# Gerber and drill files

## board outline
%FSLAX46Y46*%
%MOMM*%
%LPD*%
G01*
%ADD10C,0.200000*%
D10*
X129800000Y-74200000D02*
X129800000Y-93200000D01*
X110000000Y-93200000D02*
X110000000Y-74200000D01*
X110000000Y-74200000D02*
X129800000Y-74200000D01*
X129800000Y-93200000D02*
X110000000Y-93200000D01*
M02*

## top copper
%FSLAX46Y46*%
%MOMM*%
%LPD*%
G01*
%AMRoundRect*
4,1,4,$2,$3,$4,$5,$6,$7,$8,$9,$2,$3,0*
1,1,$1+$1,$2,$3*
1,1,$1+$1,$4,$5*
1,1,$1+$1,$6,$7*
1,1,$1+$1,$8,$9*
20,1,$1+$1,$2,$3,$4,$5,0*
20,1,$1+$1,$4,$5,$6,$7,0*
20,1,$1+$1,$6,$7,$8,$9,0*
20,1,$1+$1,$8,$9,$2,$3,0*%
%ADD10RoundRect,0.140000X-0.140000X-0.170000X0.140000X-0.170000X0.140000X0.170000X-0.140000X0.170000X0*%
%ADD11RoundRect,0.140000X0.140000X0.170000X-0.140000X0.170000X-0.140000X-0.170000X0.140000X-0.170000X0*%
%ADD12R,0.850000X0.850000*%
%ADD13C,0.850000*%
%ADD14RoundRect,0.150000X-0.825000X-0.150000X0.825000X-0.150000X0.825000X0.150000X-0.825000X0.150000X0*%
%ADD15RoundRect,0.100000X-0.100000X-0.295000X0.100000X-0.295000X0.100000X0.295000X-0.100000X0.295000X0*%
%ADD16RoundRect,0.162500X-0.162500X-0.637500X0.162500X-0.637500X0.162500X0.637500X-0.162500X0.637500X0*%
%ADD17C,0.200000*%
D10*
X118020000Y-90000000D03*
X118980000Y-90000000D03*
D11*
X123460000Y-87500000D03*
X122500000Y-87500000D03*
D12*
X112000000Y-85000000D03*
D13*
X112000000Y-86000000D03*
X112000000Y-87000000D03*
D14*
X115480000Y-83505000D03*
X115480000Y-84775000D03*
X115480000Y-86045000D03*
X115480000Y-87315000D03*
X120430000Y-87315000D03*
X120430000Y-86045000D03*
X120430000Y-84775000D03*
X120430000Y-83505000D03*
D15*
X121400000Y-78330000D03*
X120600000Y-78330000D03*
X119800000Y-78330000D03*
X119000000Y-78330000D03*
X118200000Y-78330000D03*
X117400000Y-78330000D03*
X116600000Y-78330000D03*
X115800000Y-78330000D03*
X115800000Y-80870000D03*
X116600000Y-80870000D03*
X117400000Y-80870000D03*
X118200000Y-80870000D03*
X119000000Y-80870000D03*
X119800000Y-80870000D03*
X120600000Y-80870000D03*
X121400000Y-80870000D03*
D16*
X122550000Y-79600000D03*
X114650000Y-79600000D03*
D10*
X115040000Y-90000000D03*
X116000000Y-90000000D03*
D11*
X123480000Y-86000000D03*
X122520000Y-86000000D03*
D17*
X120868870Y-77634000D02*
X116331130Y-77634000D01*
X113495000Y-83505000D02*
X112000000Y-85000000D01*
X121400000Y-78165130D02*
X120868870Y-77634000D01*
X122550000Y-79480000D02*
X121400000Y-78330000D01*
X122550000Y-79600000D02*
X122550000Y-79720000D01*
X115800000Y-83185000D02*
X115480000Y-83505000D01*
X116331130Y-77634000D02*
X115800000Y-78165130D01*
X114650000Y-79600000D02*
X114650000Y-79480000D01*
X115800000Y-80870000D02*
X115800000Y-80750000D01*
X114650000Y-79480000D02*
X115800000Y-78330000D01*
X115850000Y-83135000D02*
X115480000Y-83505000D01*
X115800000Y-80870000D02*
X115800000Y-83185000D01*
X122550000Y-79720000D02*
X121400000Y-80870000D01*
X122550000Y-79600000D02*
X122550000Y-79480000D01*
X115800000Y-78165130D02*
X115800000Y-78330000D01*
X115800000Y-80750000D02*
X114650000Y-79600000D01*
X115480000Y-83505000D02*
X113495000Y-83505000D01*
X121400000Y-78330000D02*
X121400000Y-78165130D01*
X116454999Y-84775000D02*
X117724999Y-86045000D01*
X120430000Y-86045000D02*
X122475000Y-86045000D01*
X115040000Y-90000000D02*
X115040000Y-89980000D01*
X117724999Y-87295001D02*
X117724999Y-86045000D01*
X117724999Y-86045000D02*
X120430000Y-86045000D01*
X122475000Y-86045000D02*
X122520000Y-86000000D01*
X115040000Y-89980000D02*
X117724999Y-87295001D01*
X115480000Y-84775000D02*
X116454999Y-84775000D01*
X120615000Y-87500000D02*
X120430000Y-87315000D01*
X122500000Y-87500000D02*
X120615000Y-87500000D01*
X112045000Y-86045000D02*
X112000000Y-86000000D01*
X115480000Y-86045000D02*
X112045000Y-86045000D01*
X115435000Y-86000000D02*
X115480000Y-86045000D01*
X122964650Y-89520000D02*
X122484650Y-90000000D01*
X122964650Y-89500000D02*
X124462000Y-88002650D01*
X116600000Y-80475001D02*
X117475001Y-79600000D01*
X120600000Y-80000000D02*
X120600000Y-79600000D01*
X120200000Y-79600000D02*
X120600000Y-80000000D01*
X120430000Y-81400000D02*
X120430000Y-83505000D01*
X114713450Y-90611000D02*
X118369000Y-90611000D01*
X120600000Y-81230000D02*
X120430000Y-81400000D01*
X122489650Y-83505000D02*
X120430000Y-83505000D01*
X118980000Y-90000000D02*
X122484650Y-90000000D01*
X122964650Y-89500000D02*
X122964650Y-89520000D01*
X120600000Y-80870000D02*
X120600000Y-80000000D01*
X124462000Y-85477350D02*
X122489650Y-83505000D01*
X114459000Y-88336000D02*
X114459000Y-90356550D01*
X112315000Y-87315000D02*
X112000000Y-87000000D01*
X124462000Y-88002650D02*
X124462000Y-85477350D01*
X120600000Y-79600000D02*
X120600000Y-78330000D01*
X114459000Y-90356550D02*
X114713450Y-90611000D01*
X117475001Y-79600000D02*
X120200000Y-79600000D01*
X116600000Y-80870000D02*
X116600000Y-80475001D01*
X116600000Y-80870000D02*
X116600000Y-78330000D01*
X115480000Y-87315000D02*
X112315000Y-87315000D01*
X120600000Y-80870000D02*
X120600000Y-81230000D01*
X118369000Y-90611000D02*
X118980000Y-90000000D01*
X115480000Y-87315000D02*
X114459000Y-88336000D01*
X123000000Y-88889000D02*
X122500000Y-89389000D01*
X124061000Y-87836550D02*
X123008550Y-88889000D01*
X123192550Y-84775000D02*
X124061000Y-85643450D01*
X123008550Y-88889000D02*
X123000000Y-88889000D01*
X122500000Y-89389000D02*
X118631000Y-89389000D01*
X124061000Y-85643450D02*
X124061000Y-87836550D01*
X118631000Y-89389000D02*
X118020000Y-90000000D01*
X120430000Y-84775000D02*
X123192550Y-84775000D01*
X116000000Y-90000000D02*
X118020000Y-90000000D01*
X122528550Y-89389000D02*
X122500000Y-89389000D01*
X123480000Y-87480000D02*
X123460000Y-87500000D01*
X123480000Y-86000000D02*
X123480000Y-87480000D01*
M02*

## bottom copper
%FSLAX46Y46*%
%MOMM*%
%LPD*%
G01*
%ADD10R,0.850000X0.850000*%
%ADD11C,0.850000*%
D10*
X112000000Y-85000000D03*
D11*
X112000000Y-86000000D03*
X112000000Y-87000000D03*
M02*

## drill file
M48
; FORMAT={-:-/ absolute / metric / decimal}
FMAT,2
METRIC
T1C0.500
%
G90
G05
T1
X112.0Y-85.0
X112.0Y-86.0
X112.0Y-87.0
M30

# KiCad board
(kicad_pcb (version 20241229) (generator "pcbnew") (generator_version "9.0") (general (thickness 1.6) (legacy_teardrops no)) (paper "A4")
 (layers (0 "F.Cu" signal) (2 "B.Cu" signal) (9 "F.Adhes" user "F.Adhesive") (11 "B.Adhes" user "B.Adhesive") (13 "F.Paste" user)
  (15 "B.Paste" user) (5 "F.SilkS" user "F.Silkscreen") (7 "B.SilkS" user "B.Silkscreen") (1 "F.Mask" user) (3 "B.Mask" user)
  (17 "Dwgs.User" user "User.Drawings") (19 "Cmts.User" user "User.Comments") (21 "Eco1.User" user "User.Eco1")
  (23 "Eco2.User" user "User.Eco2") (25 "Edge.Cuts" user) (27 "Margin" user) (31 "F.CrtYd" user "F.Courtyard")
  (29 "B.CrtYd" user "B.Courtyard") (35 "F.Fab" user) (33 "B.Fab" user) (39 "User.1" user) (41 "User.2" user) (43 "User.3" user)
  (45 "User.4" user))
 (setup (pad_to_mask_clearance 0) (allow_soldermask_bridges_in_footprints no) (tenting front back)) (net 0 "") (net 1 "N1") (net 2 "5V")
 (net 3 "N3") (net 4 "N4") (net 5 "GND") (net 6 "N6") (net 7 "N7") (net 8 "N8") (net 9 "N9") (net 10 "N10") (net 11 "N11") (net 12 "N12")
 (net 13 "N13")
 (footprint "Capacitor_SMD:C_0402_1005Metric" (layer "F.Cu") (at 118.5 90)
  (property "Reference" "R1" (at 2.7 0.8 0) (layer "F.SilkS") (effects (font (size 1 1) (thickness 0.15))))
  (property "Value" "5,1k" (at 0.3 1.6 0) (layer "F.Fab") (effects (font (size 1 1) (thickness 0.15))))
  (pad "1" smd roundrect (at -0.48 0) (size 0.56 0.62) (layers "F.Cu" "F.Mask" "F.Paste") (roundrect_rratio 0.25) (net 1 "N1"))
  (pad "2" smd roundrect (at 0.48 0) (size 0.56 0.62) (layers "F.Cu" "F.Mask" "F.Paste") (roundrect_rratio 0.25) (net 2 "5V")))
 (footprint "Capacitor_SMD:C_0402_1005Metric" (layer "F.Cu") (at 122.98 87.5 180)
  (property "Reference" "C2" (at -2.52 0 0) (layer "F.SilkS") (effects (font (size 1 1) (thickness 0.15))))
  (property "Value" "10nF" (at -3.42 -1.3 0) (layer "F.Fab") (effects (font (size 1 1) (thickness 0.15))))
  (pad "1" smd roundrect (at -0.48 0 180) (size 0.56 0.62) (layers "F.Cu" "F.Mask" "F.Paste") (roundrect_rratio 0.25) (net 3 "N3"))
  (pad "2" smd roundrect (at 0.48 0 180) (size 0.56 0.62) (layers "F.Cu" "F.Mask" "F.Paste") (roundrect_rratio 0.25) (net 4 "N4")))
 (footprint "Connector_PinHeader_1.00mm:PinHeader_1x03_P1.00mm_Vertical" (layer "F.Cu") (at 112 85)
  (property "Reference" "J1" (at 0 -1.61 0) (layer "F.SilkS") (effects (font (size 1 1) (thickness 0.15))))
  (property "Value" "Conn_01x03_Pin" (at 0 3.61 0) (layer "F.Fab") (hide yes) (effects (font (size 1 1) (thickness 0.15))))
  (pad "1" thru_hole rect (at 0 0) (size 0.85 0.85) (drill 0.5) (layers "*.Cu" "*.Mask") (remove_unused_layers no) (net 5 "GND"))
  (pad "2" thru_hole circle (at 0 1) (size 0.85 0.85) (drill 0.5) (layers "*.Cu" "*.Mask") (remove_unused_layers no) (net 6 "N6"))
  (pad "3" thru_hole circle (at 0 2) (size 0.85 0.85) (drill 0.5) (layers "*.Cu" "*.Mask") (remove_unused_layers no) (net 2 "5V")))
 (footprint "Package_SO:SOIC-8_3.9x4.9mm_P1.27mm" (layer "F.Cu") (at 117.955 85.41)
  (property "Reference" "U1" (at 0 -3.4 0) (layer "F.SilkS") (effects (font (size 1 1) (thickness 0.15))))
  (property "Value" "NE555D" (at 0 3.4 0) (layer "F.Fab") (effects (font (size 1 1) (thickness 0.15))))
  (pad "1" smd roundrect (at -2.475 -1.905) (size 1.95 0.6) (layers "F.Cu" "F.Mask" "F.Paste") (roundrect_rratio 0.25) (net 5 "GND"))
  (pad "2" smd roundrect (at -2.475 -0.635) (size 1.95 0.6) (layers "F.Cu" "F.Mask" "F.Paste") (roundrect_rratio 0.25) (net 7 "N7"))
  (pad "3" smd roundrect (at -2.475 0.635) (size 1.95 0.6) (layers "F.Cu" "F.Mask" "F.Paste") (roundrect_rratio 0.25) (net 6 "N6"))
  (pad "4" smd roundrect (at -2.475 1.905) (size 1.95 0.6) (layers "F.Cu" "F.Mask" "F.Paste") (roundrect_rratio 0.25) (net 2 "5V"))
  (pad "5" smd roundrect (at 2.475 1.905) (size 1.95 0.6) (layers "F.Cu" "F.Mask" "F.Paste") (roundrect_rratio 0.25) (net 4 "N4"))
  (pad "6" smd roundrect (at 2.475 0.635) (size 1.95 0.6) (layers "F.Cu" "F.Mask" "F.Paste") (roundrect_rratio 0.25) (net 7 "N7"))
  (pad "7" smd roundrect (at 2.475 -0.635) (size 1.95 0.6) (layers "F.Cu" "F.Mask" "F.Paste") (roundrect_rratio 0.25) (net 1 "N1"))
  (pad "8" smd roundrect (at 2.475 -1.905) (size 1.95 0.6) (layers "F.Cu" "F.Mask" "F.Paste") (roundrect_rratio 0.25) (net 2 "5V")))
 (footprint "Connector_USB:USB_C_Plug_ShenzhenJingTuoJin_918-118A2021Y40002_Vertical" (layer "F.Cu") (at 118.6 79.6 -90)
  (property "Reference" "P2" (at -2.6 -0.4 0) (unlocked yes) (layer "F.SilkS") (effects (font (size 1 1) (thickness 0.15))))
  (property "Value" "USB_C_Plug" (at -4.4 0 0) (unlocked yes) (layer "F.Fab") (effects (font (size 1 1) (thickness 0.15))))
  (pad "A1" smd roundrect (at -1.27 -2.8) (size 0.4 0.79) (layers "F.Cu" "F.Mask" "F.Paste") (roundrect_rratio 0.25) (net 5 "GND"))
  (pad "A4" smd roundrect (at -1.27 -2) (size 0.4 0.79) (layers "F.Cu" "F.Mask" "F.Paste") (roundrect_rratio 0.25) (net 2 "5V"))
  (pad "A5" smd roundrect (at -1.27 -1.2) (size 0.4 0.79) (layers "F.Cu" "F.Mask" "F.Paste") (roundrect_rratio 0.25) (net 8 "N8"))
  (pad "A6" smd roundrect (at -1.27 -0.4) (size 0.4 0.79) (layers "F.Cu" "F.Mask" "F.Paste") (roundrect_rratio 0.25) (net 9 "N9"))
  (pad "A7" smd roundrect (at -1.27 0.4) (size 0.4 0.79) (layers "F.Cu" "F.Mask" "F.Paste") (roundrect_rratio 0.25) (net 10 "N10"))
  (pad "A8" smd roundrect (at -1.27 1.2) (size 0.4 0.79) (layers "F.Cu" "F.Mask" "F.Paste") (roundrect_rratio 0.25) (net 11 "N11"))
  (pad "A9" smd roundrect (at -1.27 2) (size 0.4 0.79) (layers "F.Cu" "F.Mask" "F.Paste") (roundrect_rratio 0.25) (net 2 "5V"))
  (pad "A12" smd roundrect (at -1.27 2.8) (size 0.4 0.79) (layers "F.Cu" "F.Mask" "F.Paste") (roundrect_rratio 0.25) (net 5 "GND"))
  (pad "B1" smd roundrect (at 1.27 2.8) (size 0.4 0.79) (layers "F.Cu" "F.Mask" "F.Paste") (roundrect_rratio 0.25) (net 5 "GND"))
  (pad "B4" smd roundrect (at 1.27 2) (size 0.4 0.79) (layers "F.Cu" "F.Mask" "F.Paste") (roundrect_rratio 0.25) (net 2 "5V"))
  (pad "B5" smd roundrect (at 1.27 1.2) (size 0.4 0.79) (layers "F.Cu" "F.Mask" "F.Paste") (roundrect_rratio 0.25) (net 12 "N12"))
  (pad "B6" smd roundrect (at 1.27 0.4) (size 0.4 0.79) (layers "F.Cu" "F.Mask" "F.Paste") (roundrect_rratio 0.25))
  (pad "B7" smd roundrect (at 1.27 -0.4) (size 0.4 0.79) (layers "F.Cu" "F.Mask" "F.Paste") (roundrect_rratio 0.25))
  (pad "B8" smd roundrect (at 1.27 -1.2) (size 0.4 0.79) (layers "F.Cu" "F.Mask" "F.Paste") (roundrect_rratio 0.25) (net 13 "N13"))
  (pad "B9" smd roundrect (at 1.27 -2) (size 0.4 0.79) (layers "F.Cu" "F.Mask" "F.Paste") (roundrect_rratio 0.25) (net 2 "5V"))
  (pad "B12" smd roundrect (at 1.27 -2.8) (size 0.4 0.79) (layers "F.Cu" "F.Mask" "F.Paste") (roundrect_rratio 0.25) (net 5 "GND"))
  (pad "S1" smd roundrect (at 0 -3.95) (size 0.65 1.6) (layers "F.Cu" "F.Mask" "F.Paste") (roundrect_rratio 0.25) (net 5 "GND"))
  (pad "S1" smd roundrect (at 0 3.95) (size 0.65 1.6) (layers "F.Cu" "F.Mask" "F.Paste") (roundrect_rratio 0.25) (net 5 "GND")))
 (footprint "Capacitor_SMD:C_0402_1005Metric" (layer "F.Cu") (at 115.52 90)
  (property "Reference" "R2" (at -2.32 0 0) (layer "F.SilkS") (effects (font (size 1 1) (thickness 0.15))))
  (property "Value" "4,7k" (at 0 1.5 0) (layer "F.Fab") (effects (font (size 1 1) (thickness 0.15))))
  (pad "1" smd roundrect (at -0.48 0) (size 0.56 0.62) (layers "F.Cu" "F.Mask" "F.Paste") (roundrect_rratio 0.25) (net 7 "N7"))
  (pad "2" smd roundrect (at 0.48 0) (size 0.56 0.62) (layers "F.Cu" "F.Mask" "F.Paste") (roundrect_rratio 0.25) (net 1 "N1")))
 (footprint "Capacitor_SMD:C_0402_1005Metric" (layer "F.Cu") (at 123 86 180)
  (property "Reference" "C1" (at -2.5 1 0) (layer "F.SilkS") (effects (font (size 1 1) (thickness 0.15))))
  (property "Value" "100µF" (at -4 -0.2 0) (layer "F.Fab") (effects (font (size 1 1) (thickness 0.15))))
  (pad "1" smd roundrect (at -0.48 0 180) (size 0.56 0.62) (layers "F.Cu" "F.Mask" "F.Paste") (roundrect_rratio 0.25) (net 3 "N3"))
  (pad "2" smd roundrect (at 0.48 0 180) (size 0.56 0.62) (layers "F.Cu" "F.Mask" "F.Paste") (roundrect_rratio 0.25) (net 7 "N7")))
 (gr_line (start 129.8 74.2) (end 129.8 93.2) (stroke (width 0.2) (type solid)) (layer "Edge.Cuts"))
 (gr_line (start 110 93.2) (end 110 74.2) (stroke (width 0.2) (type solid)) (layer "Edge.Cuts"))
 (gr_line (start 110 74.2) (end 129.8 74.2) (stroke (width 0.2) (type solid)) (layer "Edge.Cuts"))
 (gr_line (start 129.8 93.2) (end 110 93.2) (stroke (width 0.2) (type solid)) (layer "Edge.Cuts"))
 (segment (start 120.86887 77.634) (end 116.33113 77.634) (width 0.2) (layer "F.Cu") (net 5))
 (segment (start 113.495 83.505) (end 112 85) (width 0.2) (layer "F.Cu") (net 5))
 (segment (start 121.4 78.16513) (end 120.86887 77.634) (width 0.2) (layer "F.Cu") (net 5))
 (segment (start 122.55 79.48) (end 121.4 78.33) (width 0.2) (layer "F.Cu") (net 5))
 (segment (start 122.55 79.6) (end 122.55 79.72) (width 0.2) (layer "F.Cu") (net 5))
 (segment (start 115.8 83.185) (end 115.48 83.505) (width 0.2) (layer "F.Cu") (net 5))
 (segment (start 116.33113 77.634) (end 115.8 78.16513) (width 0.2) (layer "F.Cu") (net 5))
 (segment (start 114.65 79.6) (end 114.65 79.48) (width 0.2) (layer "F.Cu") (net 5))
 (segment (start 115.8 80.87) (end 115.8 80.75) (width 0.2) (layer "F.Cu") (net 5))
 (segment (start 114.65 79.48) (end 115.8 78.33) (width 0.2) (layer "F.Cu") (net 5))
 (segment (start 115.85 83.135) (end 115.48 83.505) (width 0.2) (layer "F.Cu") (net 5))
 (segment (start 115.8 80.87) (end 115.8 83.185) (width 0.2) (layer "F.Cu") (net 5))
 (segment (start 122.55 79.72) (end 121.4 80.87) (width 0.2) (layer "F.Cu") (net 5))
 (segment (start 122.55 79.6) (end 122.55 79.48) (width 0.2) (layer "F.Cu") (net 5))
 (segment (start 115.8 78.16513) (end 115.8 78.33) (width 0.2) (layer "F.Cu") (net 5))
 (segment (start 115.8 80.75) (end 114.65 79.6) (width 0.2) (layer "F.Cu") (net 5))
 (segment (start 115.48 83.505) (end 113.495 83.505) (width 0.2) (layer "F.Cu") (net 5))
 (segment (start 121.4 78.33) (end 121.4 78.16513) (width 0.2) (layer "F.Cu") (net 5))
 (segment (start 116.454999 84.775) (end 117.724999 86.045) (width 0.2) (layer "F.Cu") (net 7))
 (segment (start 120.43 86.045) (end 122.475 86.045) (width 0.2) (layer "F.Cu") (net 7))
 (segment (start 115.04 90) (end 115.04 89.98) (width 0.2) (layer "F.Cu") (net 7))
 (segment (start 117.724999 87.295001) (end 117.724999 86.045) (width 0.2) (layer "F.Cu") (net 7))
 (segment (start 117.724999 86.045) (end 120.43 86.045) (width 0.2) (layer "F.Cu") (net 7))
 (segment (start 122.475 86.045) (end 122.52 86) (width 0.2) (layer "F.Cu") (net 7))
 (segment (start 115.04 89.98) (end 117.724999 87.295001) (width 0.2) (layer "F.Cu") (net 7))
 (segment (start 115.48 84.775) (end 116.454999 84.775) (width 0.2) (layer "F.Cu") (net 7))
 (segment (start 120.615 87.5) (end 120.43 87.315) (width 0.2) (layer "F.Cu") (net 4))
 (segment (start 122.5 87.5) (end 120.615 87.5) (width 0.2) (layer "F.Cu") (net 4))
 (segment (start 112.045 86.045) (end 112 86) (width 0.2) (layer "F.Cu") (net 6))
 (segment (start 115.48 86.045) (end 112.045 86.045) (width 0.2) (layer "F.Cu") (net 6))
 (segment (start 115.435 86) (end 115.48 86.045) (width 0.2) (layer "F.Cu") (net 6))
 (segment (start 122.96465 89.52) (end 122.48465 90) (width 0.2) (layer "F.Cu") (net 2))
 (segment (start 122.96465 89.5) (end 124.462 88.00265) (width 0.2) (layer "F.Cu") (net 2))
 (segment (start 116.6 80.475001) (end 117.475001 79.6) (width 0.2) (layer "F.Cu") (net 2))
 (segment (start 120.6 80) (end 120.6 79.6) (width 0.2) (layer "F.Cu") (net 2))
 (segment (start 120.2 79.6) (end 120.6 80) (width 0.2) (layer "F.Cu") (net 2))
 (segment (start 120.43 81.4) (end 120.43 83.505) (width 0.2) (layer "F.Cu") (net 2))
 (segment (start 114.71345 90.611) (end 118.369 90.611) (width 0.2) (layer "F.Cu") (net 2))
 (segment (start 120.6 81.23) (end 120.43 81.4) (width 0.2) (layer "F.Cu") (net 2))
 (segment (start 122.48965 83.505) (end 120.43 83.505) (width 0.2) (layer "F.Cu") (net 2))
 (segment (start 118.98 90) (end 122.48465 90) (width 0.2) (layer "F.Cu") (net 2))
 (segment (start 122.96465 89.5) (end 122.96465 89.52) (width 0.2) (layer "F.Cu") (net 2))
 (segment (start 120.6 80.87) (end 120.6 80) (width 0.2) (layer "F.Cu") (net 2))
 (segment (start 124.462 85.47735) (end 122.48965 83.505) (width 0.2) (layer "F.Cu") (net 2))
 (segment (start 114.459 88.336) (end 114.459 90.35655) (width 0.2) (layer "F.Cu") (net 2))
 (segment (start 112.315 87.315) (end 112 87) (width 0.2) (layer "F.Cu") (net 2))
 (segment (start 124.462 88.00265) (end 124.462 85.47735) (width 0.2) (layer "F.Cu") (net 2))
 (segment (start 120.6 79.6) (end 120.6 78.33) (width 0.2) (layer "F.Cu") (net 2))
 (segment (start 114.459 90.35655) (end 114.71345 90.611) (width 0.2) (layer "F.Cu") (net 2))
 (segment (start 117.475001 79.6) (end 120.2 79.6) (width 0.2) (layer "F.Cu") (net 2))
 (segment (start 116.6 80.87) (end 116.6 80.475001) (width 0.2) (layer "F.Cu") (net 2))
 (segment (start 116.6 80.87) (end 116.6 78.33) (width 0.2) (layer "F.Cu") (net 2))
 (segment (start 115.48 87.315) (end 112.315 87.315) (width 0.2) (layer "F.Cu") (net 2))
 (segment (start 120.6 80.87) (end 120.6 81.23) (width 0.2) (layer "F.Cu") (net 2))
 (segment (start 118.369 90.611) (end 118.98 90) (width 0.2) (layer "F.Cu") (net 2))
 (segment (start 115.48 87.315) (end 114.459 88.336) (width 0.2) (layer "F.Cu") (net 2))
 (segment (start 123 88.889) (end 122.5 89.389) (width 0.2) (layer "F.Cu") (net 1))
 (segment (start 124.061 87.83655) (end 123.00855 88.889) (width 0.2) (layer "F.Cu") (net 1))
 (segment (start 123.19255 84.775) (end 124.061 85.64345) (width 0.2) (layer "F.Cu") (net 1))
 (segment (start 123.00855 88.889) (end 123 88.889) (width 0.2) (layer "F.Cu") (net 1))
 (segment (start 122.5 89.389) (end 118.631 89.389) (width 0.2) (layer "F.Cu") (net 1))
 (segment (start 124.061 85.64345) (end 124.061 87.83655) (width 0.2) (layer "F.Cu") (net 1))
 (segment (start 118.631 89.389) (end 118.02 90) (width 0.2) (layer "F.Cu") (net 1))
 (segment (start 120.43 84.775) (end 123.19255 84.775) (width 0.2) (layer "F.Cu") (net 1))
 (segment (start 116 90) (end 118.02 90) (width 0.2) (layer "F.Cu") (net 1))
 (segment (start 122.52855 89.389) (end 122.5 89.389) (width 0.2) (layer "F.Cu") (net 1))
 (segment (start 123.48 87.48) (end 123.46 87.5) (width 0.2) (layer "F.Cu") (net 3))
 (segment (start 123.48 86) (end 123.48 87.48) (width 0.2) (layer "F.Cu") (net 3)))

